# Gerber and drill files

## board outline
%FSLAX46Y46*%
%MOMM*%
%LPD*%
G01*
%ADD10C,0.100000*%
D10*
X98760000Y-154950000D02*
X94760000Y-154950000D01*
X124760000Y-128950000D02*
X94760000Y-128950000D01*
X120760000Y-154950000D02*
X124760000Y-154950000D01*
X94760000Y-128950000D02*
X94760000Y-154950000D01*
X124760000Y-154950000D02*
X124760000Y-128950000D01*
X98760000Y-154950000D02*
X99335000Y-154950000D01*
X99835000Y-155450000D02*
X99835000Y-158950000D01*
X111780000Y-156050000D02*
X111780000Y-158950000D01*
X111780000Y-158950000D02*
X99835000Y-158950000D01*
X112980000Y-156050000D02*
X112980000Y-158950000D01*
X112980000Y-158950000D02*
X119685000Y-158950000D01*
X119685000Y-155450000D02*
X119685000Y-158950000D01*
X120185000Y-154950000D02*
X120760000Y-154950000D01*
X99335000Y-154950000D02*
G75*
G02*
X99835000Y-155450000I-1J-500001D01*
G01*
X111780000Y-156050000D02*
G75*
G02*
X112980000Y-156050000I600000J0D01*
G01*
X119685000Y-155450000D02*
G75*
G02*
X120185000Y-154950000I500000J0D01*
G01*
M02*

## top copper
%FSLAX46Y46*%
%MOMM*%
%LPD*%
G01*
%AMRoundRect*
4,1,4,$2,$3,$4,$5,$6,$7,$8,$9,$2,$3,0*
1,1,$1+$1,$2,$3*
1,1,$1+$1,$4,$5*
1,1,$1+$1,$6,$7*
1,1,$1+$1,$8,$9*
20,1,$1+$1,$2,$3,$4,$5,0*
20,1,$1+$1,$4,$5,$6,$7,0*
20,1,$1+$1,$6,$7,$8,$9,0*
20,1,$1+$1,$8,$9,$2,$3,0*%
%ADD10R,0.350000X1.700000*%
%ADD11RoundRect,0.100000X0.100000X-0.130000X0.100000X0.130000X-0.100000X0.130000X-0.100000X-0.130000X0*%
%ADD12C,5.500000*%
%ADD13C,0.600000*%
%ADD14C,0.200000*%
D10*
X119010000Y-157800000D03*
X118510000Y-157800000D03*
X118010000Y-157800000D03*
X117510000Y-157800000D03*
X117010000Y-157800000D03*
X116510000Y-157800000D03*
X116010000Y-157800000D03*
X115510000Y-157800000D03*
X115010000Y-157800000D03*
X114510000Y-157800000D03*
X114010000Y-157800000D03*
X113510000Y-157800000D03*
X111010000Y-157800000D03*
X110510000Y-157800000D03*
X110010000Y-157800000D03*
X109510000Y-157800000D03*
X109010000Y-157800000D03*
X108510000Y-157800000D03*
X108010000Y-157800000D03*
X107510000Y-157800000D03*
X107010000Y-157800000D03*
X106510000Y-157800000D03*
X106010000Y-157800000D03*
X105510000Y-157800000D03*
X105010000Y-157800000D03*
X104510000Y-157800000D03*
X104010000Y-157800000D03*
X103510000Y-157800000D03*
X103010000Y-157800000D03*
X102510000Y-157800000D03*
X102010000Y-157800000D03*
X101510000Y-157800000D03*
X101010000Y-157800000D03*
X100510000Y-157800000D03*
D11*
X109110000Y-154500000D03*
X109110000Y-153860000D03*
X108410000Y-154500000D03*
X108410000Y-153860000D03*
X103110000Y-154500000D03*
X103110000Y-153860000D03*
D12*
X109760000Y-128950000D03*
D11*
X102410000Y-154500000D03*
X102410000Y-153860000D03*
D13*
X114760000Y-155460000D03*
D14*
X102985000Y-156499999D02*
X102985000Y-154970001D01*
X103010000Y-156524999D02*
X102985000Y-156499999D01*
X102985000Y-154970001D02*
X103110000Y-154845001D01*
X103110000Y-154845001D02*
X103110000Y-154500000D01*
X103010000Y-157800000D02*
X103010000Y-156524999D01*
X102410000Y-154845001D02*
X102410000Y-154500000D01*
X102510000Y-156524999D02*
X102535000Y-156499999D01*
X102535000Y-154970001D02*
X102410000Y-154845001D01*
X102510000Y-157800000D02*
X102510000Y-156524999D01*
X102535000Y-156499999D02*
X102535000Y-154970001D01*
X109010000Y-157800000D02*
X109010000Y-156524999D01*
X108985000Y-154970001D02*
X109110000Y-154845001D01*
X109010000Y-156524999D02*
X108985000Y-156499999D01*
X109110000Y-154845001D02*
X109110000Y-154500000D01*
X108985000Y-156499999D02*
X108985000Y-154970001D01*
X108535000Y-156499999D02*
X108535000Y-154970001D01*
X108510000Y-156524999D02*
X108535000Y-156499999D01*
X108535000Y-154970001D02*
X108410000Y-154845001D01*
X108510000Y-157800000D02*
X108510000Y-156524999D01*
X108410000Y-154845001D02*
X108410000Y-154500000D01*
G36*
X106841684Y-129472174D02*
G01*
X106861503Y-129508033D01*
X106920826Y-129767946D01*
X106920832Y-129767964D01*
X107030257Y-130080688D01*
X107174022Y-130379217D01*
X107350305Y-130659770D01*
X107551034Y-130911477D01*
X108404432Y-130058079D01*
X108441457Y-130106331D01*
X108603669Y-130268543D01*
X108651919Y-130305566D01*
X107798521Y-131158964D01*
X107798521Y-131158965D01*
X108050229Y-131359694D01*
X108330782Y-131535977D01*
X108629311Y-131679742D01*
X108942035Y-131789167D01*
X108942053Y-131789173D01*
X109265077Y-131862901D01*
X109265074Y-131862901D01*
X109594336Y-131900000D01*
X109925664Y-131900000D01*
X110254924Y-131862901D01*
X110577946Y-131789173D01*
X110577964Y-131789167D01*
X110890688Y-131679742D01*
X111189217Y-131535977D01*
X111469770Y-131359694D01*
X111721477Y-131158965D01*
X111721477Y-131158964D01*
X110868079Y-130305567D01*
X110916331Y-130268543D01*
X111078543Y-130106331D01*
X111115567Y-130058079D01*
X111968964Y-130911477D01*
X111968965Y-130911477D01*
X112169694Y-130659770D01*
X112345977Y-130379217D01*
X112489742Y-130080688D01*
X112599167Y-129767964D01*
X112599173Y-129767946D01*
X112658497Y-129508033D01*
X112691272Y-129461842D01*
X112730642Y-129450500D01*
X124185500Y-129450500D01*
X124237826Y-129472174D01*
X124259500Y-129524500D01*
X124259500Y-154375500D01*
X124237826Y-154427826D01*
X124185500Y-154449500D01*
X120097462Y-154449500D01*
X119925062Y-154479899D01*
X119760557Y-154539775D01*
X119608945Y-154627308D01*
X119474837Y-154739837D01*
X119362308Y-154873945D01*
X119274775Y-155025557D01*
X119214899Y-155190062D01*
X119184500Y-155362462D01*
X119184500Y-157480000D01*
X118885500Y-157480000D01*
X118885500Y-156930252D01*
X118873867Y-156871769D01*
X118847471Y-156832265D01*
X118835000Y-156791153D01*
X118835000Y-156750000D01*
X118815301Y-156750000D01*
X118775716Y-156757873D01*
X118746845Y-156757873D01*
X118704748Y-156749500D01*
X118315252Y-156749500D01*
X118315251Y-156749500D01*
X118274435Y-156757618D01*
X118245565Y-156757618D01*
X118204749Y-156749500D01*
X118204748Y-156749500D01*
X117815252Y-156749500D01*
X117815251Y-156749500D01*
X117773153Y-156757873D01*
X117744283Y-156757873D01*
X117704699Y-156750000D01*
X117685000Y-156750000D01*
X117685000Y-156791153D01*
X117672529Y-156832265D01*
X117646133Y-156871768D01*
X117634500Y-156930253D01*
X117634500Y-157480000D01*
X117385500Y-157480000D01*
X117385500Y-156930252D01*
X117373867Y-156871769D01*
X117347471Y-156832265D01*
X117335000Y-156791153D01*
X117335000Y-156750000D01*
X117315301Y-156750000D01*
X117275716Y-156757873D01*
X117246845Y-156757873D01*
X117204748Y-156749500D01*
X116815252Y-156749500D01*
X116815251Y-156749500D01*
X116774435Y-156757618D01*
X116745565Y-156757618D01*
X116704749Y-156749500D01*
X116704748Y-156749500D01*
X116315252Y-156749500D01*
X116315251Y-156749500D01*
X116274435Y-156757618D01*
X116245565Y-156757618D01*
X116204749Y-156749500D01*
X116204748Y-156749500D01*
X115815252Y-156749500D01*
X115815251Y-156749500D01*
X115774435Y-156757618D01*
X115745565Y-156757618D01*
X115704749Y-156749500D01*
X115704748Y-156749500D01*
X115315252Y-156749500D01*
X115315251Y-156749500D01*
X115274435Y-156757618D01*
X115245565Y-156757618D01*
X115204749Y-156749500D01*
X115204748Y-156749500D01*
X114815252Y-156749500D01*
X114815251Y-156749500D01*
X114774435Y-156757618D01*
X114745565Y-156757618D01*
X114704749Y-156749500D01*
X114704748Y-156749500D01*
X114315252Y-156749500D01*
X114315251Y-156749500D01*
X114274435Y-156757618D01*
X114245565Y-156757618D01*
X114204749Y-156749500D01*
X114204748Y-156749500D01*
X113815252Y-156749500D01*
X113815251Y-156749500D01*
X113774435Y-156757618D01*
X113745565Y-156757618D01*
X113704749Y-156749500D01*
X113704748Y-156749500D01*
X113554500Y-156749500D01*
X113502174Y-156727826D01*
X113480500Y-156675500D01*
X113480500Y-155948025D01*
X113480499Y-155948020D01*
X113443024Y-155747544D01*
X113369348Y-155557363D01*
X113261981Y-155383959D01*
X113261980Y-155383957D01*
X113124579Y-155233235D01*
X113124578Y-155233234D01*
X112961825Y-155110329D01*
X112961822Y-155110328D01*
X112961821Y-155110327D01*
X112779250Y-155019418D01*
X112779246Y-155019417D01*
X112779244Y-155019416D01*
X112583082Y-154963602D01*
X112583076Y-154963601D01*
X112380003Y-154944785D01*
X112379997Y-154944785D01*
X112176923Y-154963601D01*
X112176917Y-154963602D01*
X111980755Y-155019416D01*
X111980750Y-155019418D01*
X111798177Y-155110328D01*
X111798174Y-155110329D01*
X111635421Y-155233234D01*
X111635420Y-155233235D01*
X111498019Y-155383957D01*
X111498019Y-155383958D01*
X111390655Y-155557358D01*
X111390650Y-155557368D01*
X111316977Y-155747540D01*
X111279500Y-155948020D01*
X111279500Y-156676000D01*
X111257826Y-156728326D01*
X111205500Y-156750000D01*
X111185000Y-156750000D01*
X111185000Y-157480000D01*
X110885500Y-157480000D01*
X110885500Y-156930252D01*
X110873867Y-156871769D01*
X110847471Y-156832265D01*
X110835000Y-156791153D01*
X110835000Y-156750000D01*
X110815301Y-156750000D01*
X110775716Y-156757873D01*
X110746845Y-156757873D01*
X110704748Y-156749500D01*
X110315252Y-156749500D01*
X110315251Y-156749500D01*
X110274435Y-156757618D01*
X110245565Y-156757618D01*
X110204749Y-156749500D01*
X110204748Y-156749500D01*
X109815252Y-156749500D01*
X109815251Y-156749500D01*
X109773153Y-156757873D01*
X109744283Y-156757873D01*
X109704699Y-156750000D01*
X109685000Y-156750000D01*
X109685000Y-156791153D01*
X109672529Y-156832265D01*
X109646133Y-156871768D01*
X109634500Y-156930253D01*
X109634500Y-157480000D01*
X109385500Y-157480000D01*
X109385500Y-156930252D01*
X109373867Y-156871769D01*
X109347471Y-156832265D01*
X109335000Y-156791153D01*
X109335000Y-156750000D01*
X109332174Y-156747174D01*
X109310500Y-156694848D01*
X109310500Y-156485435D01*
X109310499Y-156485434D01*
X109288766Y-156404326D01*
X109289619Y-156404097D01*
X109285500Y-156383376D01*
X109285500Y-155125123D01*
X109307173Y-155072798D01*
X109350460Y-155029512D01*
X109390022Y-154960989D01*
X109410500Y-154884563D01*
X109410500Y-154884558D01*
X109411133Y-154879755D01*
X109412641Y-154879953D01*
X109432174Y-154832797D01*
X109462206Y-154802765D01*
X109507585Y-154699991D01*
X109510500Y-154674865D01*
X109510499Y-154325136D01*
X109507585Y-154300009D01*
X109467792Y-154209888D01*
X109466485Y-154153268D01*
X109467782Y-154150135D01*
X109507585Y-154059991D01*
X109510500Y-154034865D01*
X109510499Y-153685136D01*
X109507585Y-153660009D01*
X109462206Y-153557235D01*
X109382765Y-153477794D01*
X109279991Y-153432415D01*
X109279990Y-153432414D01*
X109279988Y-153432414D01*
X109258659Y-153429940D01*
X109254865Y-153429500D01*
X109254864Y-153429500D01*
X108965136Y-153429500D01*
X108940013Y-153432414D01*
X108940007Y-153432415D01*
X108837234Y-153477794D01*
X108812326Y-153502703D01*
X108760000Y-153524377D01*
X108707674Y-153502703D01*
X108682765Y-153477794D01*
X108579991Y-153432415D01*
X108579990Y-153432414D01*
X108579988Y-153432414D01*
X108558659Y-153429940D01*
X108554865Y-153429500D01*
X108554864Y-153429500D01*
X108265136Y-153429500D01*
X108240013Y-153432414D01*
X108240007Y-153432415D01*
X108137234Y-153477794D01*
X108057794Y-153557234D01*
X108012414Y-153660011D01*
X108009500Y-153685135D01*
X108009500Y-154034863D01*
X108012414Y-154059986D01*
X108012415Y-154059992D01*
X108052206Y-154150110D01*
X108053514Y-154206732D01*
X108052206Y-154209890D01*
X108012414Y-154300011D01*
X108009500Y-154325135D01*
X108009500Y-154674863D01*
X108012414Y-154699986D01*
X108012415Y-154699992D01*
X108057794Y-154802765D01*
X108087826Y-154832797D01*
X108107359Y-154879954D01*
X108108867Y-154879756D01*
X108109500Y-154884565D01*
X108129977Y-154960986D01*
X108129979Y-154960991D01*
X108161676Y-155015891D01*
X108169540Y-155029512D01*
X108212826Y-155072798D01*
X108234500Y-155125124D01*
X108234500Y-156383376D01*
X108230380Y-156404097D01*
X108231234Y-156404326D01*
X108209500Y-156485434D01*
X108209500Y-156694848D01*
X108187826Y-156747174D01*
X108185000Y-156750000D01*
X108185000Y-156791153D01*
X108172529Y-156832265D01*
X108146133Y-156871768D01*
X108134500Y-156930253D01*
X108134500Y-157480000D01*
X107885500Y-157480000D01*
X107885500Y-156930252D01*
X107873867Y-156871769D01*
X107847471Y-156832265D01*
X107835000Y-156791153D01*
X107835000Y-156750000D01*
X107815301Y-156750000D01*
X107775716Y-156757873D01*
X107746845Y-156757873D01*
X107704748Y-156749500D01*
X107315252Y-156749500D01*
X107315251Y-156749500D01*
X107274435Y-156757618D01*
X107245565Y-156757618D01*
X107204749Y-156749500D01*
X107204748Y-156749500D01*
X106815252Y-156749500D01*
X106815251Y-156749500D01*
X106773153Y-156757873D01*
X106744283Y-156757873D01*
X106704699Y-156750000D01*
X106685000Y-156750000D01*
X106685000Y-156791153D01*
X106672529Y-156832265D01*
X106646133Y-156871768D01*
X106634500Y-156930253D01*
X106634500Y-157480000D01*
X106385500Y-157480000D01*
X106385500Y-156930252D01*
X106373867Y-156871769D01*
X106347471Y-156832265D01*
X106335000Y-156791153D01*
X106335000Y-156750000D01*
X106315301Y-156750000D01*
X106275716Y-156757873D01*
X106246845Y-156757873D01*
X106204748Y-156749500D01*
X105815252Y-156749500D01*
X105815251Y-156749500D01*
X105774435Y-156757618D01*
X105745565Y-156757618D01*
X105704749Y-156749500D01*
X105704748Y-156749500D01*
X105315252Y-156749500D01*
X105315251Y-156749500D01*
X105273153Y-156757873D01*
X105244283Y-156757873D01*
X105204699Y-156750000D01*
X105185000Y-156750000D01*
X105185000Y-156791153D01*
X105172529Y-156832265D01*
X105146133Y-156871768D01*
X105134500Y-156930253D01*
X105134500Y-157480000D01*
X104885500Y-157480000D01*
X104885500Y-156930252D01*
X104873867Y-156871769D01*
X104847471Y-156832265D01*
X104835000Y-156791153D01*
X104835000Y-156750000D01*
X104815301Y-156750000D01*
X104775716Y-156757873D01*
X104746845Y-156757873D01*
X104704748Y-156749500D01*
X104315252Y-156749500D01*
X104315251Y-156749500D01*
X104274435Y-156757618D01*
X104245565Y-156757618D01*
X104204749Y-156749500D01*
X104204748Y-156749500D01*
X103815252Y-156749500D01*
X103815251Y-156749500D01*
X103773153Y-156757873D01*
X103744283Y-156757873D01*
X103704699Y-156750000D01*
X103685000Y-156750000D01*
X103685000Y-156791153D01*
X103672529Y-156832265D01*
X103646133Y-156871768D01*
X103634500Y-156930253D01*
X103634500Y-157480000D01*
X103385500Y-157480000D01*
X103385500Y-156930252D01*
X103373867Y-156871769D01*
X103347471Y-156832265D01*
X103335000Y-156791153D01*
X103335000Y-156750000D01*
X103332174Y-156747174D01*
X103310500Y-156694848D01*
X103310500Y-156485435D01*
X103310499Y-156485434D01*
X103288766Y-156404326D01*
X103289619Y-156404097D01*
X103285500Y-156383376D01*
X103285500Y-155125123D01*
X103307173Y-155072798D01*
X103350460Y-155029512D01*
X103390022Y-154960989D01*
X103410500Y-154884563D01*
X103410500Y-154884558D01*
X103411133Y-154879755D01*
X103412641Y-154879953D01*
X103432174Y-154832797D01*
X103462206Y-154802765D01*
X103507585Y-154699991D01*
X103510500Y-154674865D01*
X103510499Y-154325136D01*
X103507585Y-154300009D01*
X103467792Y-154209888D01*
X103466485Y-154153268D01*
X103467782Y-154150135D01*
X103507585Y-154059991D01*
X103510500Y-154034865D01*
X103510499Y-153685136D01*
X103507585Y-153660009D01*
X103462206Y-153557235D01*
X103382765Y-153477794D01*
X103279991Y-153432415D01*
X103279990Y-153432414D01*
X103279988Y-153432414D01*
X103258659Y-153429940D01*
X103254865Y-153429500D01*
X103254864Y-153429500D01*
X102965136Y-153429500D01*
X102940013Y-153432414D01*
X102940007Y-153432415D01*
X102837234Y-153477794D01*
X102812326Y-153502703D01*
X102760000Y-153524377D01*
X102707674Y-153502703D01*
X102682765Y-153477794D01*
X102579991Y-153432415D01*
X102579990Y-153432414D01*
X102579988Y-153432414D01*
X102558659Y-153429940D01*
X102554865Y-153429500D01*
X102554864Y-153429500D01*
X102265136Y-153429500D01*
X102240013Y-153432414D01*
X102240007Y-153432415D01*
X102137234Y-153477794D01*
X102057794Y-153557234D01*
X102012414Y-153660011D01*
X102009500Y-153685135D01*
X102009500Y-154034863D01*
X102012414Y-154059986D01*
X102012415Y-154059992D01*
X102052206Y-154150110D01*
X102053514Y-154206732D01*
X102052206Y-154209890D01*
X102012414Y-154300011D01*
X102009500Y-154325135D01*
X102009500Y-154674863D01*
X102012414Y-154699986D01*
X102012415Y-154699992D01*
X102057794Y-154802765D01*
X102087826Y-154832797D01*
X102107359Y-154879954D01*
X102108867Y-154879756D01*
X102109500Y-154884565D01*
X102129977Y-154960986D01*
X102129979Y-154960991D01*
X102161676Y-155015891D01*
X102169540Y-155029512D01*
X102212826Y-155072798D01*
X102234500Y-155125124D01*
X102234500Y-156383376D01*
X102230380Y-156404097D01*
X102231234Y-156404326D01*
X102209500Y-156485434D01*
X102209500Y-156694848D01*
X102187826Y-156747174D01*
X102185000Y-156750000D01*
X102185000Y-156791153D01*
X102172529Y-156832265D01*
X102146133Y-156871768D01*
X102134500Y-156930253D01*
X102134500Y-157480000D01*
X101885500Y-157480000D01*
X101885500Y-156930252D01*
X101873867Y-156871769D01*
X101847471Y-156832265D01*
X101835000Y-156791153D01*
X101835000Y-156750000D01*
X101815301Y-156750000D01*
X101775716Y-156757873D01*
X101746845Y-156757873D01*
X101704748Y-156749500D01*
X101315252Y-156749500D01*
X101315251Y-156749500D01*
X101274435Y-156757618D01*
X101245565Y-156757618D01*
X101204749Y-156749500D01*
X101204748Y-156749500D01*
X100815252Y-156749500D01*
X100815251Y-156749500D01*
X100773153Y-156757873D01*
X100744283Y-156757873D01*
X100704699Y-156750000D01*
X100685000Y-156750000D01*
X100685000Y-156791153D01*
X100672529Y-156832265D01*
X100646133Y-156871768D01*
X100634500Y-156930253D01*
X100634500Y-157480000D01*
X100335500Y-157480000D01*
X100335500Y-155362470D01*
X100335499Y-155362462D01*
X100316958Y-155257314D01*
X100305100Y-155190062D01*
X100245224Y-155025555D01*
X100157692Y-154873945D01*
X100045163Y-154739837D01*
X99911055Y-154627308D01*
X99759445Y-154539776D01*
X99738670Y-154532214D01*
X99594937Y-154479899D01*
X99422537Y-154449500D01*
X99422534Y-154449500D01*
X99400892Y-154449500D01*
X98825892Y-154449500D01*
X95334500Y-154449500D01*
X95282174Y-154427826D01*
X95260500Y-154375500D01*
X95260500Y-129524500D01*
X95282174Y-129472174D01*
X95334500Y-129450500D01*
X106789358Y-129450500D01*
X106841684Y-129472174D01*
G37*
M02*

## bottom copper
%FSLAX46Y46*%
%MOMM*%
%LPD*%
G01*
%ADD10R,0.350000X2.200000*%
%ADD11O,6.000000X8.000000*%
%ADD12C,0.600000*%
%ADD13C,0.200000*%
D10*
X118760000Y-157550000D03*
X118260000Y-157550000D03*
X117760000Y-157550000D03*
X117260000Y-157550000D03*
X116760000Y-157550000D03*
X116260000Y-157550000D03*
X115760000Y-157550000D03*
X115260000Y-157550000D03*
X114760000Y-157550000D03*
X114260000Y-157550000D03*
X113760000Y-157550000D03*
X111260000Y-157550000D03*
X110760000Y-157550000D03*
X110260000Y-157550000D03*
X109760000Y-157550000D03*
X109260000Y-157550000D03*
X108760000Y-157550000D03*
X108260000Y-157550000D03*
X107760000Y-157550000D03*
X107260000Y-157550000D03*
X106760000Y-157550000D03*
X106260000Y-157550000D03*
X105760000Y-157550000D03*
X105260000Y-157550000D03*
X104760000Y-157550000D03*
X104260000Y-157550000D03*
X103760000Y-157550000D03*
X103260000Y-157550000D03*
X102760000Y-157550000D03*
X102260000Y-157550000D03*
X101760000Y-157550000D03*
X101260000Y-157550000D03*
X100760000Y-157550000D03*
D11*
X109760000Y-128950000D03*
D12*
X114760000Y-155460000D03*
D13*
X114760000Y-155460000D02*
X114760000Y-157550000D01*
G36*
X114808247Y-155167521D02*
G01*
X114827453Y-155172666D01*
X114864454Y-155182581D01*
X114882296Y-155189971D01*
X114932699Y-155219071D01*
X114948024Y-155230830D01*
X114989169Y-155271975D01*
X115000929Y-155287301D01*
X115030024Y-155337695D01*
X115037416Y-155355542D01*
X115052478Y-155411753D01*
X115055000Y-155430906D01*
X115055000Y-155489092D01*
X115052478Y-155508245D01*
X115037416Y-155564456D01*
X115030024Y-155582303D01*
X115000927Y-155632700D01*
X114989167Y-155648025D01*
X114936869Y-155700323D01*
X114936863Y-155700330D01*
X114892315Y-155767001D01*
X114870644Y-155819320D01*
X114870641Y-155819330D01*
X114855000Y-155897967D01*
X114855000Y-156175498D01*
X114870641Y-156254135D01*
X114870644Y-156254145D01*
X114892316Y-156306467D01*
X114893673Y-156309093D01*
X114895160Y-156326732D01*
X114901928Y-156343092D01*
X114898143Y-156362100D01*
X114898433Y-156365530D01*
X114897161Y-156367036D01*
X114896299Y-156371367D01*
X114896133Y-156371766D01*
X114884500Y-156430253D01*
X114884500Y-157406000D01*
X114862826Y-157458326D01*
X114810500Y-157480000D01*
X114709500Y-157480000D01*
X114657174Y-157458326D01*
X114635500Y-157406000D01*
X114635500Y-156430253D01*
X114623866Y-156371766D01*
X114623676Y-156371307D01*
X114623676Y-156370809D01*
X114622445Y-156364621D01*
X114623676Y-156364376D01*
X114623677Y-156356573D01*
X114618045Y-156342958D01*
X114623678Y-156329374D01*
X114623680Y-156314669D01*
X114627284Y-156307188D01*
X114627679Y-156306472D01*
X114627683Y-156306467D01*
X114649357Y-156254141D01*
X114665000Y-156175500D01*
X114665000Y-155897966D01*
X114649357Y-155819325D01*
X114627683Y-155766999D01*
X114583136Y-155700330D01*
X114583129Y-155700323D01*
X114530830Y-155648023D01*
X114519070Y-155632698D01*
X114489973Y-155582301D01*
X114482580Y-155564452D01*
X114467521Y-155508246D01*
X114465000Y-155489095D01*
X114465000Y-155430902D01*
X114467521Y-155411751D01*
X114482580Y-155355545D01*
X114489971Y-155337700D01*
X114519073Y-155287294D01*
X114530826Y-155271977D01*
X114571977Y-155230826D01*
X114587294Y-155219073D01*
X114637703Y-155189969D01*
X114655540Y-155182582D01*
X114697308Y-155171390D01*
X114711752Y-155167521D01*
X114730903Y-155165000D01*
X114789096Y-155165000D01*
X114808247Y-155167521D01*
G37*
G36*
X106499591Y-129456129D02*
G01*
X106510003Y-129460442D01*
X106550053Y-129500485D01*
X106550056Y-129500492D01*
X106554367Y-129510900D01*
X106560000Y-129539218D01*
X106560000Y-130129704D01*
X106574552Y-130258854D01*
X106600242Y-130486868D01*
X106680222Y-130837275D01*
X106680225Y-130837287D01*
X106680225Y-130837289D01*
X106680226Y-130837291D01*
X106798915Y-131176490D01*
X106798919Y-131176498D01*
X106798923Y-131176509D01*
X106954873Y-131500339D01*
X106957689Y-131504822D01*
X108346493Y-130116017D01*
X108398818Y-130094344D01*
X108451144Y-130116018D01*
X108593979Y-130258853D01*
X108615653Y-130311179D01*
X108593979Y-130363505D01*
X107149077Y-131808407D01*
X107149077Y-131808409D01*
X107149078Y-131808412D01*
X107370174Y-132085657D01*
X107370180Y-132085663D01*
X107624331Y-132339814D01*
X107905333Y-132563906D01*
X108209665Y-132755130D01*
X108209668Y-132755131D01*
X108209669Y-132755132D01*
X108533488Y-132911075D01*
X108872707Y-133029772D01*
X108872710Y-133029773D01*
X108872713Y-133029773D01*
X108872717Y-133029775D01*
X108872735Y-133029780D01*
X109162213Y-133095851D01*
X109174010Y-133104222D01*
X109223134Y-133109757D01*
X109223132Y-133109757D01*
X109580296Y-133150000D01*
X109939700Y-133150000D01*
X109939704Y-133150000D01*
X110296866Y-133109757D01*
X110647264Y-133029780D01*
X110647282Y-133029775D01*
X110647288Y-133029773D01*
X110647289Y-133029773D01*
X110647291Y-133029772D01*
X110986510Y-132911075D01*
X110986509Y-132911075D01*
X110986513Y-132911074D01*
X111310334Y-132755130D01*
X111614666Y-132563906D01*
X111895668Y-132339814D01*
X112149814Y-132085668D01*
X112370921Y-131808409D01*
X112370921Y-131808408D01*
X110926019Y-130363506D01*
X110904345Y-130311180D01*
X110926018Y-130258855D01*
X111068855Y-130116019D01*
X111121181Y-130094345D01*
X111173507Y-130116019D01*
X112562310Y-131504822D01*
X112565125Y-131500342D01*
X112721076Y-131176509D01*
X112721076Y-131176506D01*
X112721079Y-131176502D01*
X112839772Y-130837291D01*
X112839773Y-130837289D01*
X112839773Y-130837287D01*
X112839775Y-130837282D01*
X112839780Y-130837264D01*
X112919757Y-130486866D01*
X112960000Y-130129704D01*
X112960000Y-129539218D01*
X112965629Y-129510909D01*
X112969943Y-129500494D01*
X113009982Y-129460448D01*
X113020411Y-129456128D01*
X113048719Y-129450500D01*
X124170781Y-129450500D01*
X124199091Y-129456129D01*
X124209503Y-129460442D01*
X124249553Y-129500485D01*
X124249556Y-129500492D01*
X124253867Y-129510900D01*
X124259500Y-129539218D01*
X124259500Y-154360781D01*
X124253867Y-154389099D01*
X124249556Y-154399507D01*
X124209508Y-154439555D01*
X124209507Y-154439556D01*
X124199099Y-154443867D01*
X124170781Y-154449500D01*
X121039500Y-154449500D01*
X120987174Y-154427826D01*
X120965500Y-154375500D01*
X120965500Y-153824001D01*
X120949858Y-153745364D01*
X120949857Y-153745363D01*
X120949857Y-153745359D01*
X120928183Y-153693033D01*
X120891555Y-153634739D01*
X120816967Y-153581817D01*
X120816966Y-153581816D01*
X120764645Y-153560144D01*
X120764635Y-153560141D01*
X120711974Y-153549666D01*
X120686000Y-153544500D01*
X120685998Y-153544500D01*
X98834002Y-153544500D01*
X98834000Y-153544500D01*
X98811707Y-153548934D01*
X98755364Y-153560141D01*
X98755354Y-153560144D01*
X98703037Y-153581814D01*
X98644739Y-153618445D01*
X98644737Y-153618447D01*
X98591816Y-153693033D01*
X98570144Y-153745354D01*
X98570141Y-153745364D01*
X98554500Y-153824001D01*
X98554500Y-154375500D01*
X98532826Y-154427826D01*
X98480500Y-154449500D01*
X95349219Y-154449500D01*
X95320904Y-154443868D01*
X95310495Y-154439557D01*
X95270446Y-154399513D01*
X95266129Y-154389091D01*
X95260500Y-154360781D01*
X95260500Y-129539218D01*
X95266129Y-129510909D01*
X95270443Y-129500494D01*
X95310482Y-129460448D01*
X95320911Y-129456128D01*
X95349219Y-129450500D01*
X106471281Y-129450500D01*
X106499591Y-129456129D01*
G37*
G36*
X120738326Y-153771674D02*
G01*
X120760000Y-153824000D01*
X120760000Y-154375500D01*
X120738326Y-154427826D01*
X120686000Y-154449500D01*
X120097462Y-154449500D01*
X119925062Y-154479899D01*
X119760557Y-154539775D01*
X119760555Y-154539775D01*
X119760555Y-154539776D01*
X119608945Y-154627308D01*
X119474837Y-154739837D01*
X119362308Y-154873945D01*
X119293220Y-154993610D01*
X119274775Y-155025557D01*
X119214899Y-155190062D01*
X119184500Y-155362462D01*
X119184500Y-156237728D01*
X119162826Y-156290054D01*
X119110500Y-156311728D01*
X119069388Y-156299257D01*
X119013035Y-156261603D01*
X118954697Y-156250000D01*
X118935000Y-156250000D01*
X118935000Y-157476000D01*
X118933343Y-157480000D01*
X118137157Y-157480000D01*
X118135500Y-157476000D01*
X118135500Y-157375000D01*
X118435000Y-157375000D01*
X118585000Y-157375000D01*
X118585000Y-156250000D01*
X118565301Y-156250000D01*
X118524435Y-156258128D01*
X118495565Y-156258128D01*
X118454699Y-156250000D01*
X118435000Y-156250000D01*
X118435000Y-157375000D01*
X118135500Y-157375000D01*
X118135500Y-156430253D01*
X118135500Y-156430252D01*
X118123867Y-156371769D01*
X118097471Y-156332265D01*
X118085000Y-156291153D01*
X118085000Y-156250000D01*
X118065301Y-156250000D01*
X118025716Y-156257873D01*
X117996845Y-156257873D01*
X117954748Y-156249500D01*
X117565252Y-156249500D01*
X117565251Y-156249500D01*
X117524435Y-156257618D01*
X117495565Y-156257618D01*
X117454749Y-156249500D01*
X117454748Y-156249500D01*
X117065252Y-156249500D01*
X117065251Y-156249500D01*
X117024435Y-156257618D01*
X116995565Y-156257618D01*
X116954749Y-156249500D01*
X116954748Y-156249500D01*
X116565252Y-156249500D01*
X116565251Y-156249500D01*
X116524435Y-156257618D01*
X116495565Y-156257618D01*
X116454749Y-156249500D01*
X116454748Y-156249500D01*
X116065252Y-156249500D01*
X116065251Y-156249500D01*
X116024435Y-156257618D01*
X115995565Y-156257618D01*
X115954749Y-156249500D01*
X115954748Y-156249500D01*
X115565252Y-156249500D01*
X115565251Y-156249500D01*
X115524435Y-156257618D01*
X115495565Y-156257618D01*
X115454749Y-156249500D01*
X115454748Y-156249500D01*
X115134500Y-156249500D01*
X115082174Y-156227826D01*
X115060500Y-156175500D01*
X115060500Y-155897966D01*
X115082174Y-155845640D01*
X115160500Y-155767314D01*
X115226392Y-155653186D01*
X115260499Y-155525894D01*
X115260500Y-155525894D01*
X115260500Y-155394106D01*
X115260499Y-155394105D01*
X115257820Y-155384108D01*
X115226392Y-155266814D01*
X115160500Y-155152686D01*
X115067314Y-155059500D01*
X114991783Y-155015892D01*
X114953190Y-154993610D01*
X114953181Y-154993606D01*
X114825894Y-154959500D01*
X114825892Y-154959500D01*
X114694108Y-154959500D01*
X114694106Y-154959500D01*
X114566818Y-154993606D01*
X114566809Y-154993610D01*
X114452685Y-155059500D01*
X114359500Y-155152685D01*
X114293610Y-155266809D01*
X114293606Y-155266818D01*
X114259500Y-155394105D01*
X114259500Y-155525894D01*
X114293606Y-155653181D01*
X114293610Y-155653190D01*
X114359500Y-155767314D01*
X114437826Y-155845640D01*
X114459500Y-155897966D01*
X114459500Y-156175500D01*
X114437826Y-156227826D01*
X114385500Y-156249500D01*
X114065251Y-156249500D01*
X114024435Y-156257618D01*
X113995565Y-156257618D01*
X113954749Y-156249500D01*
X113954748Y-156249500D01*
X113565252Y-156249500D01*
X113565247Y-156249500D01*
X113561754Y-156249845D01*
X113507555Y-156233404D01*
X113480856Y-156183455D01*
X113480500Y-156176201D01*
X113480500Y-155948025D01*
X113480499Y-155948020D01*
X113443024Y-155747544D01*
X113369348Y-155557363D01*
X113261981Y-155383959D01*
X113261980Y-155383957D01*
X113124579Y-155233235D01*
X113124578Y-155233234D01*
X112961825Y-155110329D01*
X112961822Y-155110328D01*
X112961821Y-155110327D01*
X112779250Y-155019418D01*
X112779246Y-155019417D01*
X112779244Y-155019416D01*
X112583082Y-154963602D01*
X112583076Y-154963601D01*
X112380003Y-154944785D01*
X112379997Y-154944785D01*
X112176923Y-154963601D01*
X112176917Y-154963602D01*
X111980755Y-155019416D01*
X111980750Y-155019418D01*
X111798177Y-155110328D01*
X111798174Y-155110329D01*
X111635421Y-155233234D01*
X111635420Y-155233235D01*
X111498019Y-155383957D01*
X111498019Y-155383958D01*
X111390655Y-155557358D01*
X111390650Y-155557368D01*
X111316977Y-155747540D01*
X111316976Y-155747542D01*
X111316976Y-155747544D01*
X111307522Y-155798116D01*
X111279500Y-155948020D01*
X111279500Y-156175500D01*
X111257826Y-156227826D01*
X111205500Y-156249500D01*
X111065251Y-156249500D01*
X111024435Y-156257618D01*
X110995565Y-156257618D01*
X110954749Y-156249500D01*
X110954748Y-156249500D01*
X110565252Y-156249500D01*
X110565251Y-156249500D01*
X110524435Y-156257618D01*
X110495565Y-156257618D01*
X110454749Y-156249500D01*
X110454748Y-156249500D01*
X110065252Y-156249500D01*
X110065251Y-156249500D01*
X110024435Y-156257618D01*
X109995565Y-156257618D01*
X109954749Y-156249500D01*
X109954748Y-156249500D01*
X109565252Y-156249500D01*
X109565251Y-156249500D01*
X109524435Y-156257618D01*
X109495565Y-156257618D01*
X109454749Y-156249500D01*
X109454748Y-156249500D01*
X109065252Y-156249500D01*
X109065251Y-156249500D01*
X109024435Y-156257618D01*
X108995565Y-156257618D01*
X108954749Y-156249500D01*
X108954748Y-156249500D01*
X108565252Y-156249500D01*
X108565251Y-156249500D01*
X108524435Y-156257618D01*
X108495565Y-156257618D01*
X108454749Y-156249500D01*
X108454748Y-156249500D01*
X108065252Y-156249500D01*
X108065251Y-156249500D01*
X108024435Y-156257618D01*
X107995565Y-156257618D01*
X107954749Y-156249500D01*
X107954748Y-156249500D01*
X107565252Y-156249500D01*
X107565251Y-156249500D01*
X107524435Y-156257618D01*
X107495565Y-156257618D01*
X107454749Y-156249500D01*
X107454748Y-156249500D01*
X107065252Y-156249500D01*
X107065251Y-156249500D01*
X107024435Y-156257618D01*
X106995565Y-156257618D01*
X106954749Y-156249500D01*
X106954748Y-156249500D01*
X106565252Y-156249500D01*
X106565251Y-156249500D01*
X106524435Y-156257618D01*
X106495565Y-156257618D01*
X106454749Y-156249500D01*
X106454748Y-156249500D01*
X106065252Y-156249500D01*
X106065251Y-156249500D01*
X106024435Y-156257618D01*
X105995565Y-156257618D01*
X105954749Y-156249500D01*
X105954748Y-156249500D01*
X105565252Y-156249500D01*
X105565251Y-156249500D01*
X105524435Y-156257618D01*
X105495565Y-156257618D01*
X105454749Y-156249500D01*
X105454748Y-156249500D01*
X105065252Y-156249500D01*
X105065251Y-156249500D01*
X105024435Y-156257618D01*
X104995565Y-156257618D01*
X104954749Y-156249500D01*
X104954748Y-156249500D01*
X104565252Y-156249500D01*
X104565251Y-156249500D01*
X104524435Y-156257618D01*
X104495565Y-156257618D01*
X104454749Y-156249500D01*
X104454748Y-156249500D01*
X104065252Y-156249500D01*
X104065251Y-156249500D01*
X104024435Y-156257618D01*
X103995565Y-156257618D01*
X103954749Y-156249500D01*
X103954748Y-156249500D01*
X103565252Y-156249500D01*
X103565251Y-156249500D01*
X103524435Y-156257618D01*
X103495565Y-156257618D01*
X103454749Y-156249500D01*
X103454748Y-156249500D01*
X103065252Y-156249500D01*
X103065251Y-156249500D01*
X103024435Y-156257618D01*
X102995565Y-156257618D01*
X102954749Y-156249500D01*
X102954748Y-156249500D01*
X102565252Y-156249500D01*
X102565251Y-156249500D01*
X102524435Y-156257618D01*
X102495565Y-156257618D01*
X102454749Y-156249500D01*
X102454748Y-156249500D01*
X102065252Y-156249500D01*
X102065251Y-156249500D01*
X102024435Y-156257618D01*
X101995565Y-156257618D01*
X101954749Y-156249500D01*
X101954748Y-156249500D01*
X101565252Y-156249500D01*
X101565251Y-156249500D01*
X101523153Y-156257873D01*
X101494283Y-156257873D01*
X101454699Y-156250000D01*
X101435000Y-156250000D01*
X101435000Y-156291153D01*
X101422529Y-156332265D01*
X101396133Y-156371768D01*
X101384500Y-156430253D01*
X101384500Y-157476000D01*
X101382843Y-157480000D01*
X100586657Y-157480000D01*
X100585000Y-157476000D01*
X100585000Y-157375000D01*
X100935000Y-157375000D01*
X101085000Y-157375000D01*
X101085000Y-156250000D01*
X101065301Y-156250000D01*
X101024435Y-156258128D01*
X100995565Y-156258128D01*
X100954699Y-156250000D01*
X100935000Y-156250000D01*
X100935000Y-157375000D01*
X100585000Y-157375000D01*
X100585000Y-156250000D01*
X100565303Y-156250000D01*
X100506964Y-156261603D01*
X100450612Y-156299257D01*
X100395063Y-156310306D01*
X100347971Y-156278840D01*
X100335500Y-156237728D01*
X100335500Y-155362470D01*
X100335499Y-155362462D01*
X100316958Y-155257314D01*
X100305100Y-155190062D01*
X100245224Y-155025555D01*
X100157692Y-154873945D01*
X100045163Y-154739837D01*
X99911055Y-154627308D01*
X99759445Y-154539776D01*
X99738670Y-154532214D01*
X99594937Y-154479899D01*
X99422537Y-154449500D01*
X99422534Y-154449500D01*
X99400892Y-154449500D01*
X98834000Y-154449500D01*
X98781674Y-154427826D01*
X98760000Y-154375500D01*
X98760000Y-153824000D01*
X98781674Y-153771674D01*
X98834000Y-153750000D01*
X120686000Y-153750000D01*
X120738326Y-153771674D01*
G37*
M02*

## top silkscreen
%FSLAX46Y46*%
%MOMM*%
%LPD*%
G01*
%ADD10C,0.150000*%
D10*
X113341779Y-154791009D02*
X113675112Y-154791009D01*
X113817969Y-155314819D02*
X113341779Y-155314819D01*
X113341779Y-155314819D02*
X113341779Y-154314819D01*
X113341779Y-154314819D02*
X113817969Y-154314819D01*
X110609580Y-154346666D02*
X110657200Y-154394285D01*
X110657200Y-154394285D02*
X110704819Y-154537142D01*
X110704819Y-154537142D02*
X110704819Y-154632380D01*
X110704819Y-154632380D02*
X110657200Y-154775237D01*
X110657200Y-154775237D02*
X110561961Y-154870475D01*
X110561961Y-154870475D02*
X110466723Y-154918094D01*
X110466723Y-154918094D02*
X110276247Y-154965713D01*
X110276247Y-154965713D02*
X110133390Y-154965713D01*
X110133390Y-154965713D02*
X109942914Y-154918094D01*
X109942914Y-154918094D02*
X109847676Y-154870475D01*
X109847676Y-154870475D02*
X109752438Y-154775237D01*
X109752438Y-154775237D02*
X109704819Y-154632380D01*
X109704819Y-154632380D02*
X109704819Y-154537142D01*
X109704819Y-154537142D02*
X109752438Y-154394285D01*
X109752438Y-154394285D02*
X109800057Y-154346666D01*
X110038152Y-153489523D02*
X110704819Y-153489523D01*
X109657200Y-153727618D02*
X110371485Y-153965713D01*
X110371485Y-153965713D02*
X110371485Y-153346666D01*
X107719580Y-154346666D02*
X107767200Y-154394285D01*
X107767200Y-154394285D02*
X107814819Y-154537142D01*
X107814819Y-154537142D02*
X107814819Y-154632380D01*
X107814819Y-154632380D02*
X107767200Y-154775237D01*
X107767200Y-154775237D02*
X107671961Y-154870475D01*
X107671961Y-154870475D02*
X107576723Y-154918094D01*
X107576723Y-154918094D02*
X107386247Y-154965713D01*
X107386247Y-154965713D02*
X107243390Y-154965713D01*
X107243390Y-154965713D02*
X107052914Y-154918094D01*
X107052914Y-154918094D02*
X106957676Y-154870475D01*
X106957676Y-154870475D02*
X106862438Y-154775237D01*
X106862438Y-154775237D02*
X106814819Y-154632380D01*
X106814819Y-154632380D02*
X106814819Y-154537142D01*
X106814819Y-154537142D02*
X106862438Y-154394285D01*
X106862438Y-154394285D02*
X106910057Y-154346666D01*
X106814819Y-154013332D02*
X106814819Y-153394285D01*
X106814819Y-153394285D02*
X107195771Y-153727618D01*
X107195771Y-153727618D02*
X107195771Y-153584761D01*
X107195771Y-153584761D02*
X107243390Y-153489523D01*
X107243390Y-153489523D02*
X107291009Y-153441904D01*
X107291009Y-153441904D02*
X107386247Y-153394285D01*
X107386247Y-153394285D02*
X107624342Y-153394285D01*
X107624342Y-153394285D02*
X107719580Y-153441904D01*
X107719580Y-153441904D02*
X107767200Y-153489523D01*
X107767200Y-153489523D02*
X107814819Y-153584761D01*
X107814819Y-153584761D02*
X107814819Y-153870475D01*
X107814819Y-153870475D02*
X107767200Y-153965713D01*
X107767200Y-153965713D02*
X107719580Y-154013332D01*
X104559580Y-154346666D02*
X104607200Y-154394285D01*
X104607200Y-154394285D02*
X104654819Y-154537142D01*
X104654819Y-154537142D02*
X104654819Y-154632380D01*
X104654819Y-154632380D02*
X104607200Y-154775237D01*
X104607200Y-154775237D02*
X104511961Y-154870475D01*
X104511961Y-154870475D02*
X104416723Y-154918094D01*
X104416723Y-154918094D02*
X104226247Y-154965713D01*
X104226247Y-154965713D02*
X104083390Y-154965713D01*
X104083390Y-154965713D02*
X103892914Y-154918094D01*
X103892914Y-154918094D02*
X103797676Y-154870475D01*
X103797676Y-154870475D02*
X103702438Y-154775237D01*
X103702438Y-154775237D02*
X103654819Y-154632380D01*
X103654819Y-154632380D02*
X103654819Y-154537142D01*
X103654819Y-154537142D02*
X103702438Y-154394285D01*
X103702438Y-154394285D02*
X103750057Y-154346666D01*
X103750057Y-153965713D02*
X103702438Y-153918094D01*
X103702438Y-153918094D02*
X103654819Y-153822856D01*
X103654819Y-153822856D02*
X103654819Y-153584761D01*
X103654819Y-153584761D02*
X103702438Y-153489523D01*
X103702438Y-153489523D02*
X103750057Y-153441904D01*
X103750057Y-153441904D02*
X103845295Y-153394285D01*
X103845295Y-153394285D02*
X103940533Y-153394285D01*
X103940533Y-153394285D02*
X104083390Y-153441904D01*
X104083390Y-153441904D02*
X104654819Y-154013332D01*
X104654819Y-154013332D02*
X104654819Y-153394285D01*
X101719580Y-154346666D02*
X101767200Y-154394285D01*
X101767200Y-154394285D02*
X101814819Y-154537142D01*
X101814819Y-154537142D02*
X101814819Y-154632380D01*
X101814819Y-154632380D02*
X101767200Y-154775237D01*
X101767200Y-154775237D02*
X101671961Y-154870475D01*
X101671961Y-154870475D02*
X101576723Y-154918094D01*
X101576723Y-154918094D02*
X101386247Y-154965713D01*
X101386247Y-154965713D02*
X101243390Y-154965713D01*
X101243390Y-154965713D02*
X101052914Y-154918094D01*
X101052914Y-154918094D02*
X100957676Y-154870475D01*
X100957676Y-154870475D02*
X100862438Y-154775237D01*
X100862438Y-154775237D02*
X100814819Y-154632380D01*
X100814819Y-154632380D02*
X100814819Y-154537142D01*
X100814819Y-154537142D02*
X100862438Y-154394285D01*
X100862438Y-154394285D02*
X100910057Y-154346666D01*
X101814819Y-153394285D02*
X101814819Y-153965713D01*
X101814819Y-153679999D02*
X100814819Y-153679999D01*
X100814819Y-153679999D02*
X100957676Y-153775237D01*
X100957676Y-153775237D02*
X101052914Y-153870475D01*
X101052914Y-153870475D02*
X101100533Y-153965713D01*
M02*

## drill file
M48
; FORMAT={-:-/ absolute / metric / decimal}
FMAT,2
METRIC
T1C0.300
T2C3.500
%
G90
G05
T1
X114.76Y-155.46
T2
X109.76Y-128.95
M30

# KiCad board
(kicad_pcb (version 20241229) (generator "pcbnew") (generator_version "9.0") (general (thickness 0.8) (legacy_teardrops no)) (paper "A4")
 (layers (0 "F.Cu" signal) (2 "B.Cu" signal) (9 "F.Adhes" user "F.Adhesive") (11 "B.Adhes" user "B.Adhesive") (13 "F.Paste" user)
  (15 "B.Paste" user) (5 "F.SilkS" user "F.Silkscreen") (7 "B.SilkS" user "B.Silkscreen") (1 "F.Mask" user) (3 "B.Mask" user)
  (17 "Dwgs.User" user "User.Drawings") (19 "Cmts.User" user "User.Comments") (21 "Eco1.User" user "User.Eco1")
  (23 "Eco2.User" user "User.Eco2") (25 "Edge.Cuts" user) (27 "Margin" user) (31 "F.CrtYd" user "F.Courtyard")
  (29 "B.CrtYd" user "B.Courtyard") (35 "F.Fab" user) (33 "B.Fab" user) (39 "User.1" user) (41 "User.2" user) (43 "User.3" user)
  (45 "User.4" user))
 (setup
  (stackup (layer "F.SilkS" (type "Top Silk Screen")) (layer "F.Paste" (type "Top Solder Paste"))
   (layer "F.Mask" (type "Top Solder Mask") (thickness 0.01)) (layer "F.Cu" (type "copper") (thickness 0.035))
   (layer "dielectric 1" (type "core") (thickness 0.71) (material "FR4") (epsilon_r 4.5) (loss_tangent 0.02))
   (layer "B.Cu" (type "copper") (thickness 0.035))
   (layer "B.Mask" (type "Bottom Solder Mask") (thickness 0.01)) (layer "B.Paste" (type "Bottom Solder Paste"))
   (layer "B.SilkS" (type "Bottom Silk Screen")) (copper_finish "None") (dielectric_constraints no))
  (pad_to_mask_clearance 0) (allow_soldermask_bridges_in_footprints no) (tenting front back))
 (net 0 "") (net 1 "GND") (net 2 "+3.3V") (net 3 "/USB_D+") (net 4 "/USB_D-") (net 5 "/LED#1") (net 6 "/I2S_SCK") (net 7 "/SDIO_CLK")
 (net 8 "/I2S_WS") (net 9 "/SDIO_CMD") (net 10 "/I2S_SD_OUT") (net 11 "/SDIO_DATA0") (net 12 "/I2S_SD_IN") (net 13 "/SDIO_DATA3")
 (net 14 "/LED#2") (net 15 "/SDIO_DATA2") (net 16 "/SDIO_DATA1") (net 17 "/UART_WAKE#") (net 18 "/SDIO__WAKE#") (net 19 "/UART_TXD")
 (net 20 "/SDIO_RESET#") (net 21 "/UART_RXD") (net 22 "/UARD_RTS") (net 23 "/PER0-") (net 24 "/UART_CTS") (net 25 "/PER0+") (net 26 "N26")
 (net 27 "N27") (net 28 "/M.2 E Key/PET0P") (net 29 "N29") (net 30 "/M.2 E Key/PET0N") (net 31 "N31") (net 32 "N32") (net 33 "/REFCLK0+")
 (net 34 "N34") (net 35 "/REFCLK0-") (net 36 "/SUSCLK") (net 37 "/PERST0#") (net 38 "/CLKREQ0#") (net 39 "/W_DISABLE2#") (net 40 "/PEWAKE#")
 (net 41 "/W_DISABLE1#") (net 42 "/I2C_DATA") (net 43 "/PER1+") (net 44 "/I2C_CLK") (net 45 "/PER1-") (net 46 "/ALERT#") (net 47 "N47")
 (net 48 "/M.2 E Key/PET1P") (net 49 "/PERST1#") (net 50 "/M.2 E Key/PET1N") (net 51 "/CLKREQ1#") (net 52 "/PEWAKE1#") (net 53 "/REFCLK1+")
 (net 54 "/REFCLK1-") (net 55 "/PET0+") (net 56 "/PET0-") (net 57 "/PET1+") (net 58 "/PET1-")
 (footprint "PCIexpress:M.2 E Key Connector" (layer "F.Cu") (at 109.76 157.84)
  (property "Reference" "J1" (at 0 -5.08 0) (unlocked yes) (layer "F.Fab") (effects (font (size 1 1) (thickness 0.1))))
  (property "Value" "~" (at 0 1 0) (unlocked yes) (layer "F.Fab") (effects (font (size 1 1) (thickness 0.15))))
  (fp_line (start -11 -2.89) (end -10.425 -2.89) (stroke (width 0.1) (type default)) (layer "Edge.Cuts"))
  (fp_line (start -9.925 -2.39) (end -9.925 1.11) (stroke (width 0.1) (type default)) (layer "Edge.Cuts"))
  (fp_line (start 2.02 -1.79) (end 2.02 1.11) (stroke (width 0.1) (type default)) (layer "Edge.Cuts"))
  (fp_line (start 2.02 1.11) (end -9.925 1.11) (stroke (width 0.1) (type default)) (layer "Edge.Cuts"))
  (fp_line (start 3.22 -1.79) (end 3.22 1.11) (stroke (width 0.1) (type default)) (layer "Edge.Cuts"))
  (fp_line (start 3.22 1.11) (end 9.925 1.11) (stroke (width 0.1) (type default)) (layer "Edge.Cuts"))
  (fp_line (start 9.925 -2.39) (end 9.925 1.11) (stroke (width 0.1) (type default)) (layer "Edge.Cuts"))
  (fp_line (start 10.425 -2.89) (end 11 -2.89) (stroke (width 0.1) (type default)) (layer "Edge.Cuts"))
  (fp_arc (start -10.425 -2.89) (mid -10.071447 -2.743553) (end -9.925 -2.39) (stroke (width 0.1) (type default)) (layer "Edge.Cuts"))
  (fp_arc (start 2.02 -1.79) (mid 2.62 -2.39) (end 3.22 -1.79) (stroke (width 0.1) (type default)) (layer "Edge.Cuts"))
  (fp_arc (start 9.925 -2.39) (mid 10.071447 -2.743553) (end 10.425 -2.89) (stroke (width 0.1) (type default)) (layer "Edge.Cuts"))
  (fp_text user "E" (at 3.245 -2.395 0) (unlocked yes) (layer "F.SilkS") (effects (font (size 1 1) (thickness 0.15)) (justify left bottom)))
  (pad "1" smd rect (at 9.25 -0.04 180) (size 0.35 1.7) (layers "F.Cu") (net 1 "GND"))
  (pad "2" smd rect (at 9 -0.29 180) (size 0.35 2.2) (layers "B.Cu") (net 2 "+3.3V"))
  (pad "3" smd rect (at 8.75 -0.04 180) (size 0.35 1.7) (layers "F.Cu") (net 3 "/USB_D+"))
  (pad "4" smd rect (at 8.5 -0.29 180) (size 0.35 2.2) (layers "B.Cu") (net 2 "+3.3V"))
  (pad "5" smd rect (at 8.25 -0.04 180) (size 0.35 1.7) (layers "F.Cu") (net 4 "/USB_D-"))
  (pad "6" smd rect (at 8 -0.29 180) (size 0.35 2.2) (layers "B.Cu") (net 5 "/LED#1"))
  (pad "7" smd rect (at 7.75 -0.04 180) (size 0.35 1.7) (layers "F.Cu") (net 1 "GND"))
  (pad "8" smd rect (at 7.5 -0.29 180) (size 0.35 2.2) (layers "B.Cu") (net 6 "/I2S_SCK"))
  (pad "9" smd rect (at 7.25 -0.04 180) (size 0.35 1.7) (layers "F.Cu") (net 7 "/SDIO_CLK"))
  (pad "10" smd rect (at 7 -0.29 180) (size 0.35 2.2) (layers "B.Cu") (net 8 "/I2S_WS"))
  (pad "11" smd rect (at 6.75 -0.04 180) (size 0.35 1.7) (layers "F.Cu") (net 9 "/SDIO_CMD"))
  (pad "12" smd rect (at 6.5 -0.29 180) (size 0.35 2.2) (layers "B.Cu") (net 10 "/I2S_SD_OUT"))
  (pad "13" smd rect (at 6.25 -0.04 180) (size 0.35 1.7) (layers "F.Cu") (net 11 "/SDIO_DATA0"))
  (pad "14" smd rect (at 6 -0.29 180) (size 0.35 2.2) (layers "B.Cu") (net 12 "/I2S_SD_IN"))
  (pad "15" smd rect (at 5.75 -0.04 180) (size 0.35 1.7) (layers "F.Cu") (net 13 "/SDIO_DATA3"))
  (pad "16" smd rect (at 5.5 -0.29 180) (size 0.35 2.2) (layers "B.Cu") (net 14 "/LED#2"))
  (pad "17" smd rect (at 5.25 -0.04 180) (size 0.35 1.7) (layers "F.Cu") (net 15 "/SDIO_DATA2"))
  (pad "18" smd rect (at 5 -0.29 180) (size 0.35 2.2) (layers "B.Cu") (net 1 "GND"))
  (pad "19" smd rect (at 4.75 -0.04 180) (size 0.35 1.7) (layers "F.Cu") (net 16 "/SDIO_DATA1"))
  (pad "20" smd rect (at 4.5 -0.29 180) (size 0.35 2.2) (layers "B.Cu") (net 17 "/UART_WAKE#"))
  (pad "21" smd rect (at 4.25 -0.04 180) (size 0.35 1.7) (layers "F.Cu") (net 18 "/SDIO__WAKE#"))
  (pad "22" smd rect (at 4 -0.29 180) (size 0.35 2.2) (layers "B.Cu") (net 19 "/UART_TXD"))
  (pad "23" smd rect (at 3.75 -0.04 180) (size 0.35 1.7) (layers "F.Cu") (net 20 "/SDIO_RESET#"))
  (pad "32" smd rect (at 1.5 -0.29 180) (size 0.35 2.2) (layers "B.Cu") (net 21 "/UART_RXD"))
  (pad "33" smd rect (at 1.25 -0.04 180) (size 0.35 1.7) (layers "F.Cu") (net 1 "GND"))
  (pad "34" smd rect (at 1 -0.29 180) (size 0.35 2.2) (layers "B.Cu") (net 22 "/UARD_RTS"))
  (pad "35" smd rect (at 0.75 -0.04 180) (size 0.35 1.7) (layers "F.Cu") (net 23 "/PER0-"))
  (pad "36" smd rect (at 0.5 -0.29 180) (size 0.35 2.2) (layers "B.Cu") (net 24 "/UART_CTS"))
  (pad "37" smd rect (at 0.25 -0.04 180) (size 0.35 1.7) (layers "F.Cu") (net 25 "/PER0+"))
  (pad "38" smd rect (at 0 -0.29 180) (size 0.35 2.2) (layers "B.Cu") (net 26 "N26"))
  (pad "39" smd rect (at -0.25 -0.04 180) (size 0.35 1.7) (layers "F.Cu") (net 1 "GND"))
  (pad "40" smd rect (at -0.5 -0.29 180) (size 0.35 2.2) (layers "B.Cu") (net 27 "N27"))
  (pad "41" smd rect (at -0.75 -0.04 180) (size 0.35 1.7) (layers "F.Cu") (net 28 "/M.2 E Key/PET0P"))
  (pad "42" smd rect (at -1 -0.29 180) (size 0.35 2.2) (layers "B.Cu") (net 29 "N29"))
  (pad "43" smd rect (at -1.25 -0.04 180) (size 0.35 1.7) (layers "F.Cu") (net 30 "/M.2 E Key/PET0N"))
  (pad "44" smd rect (at -1.5 -0.29 180) (size 0.35 2.2) (layers "B.Cu") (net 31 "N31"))
  (pad "45" smd rect (at -1.75 -0.04 180) (size 0.35 1.7) (layers "F.Cu") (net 1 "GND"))
  (pad "46" smd rect (at -2 -0.29 180) (size 0.35 2.2) (layers "B.Cu") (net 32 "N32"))
  (pad "47" smd rect (at -2.25 -0.04 180) (size 0.35 1.7) (layers "F.Cu") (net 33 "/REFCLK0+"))
  (pad "48" smd rect (at -2.5 -0.29 180) (size 0.35 2.2) (layers "B.Cu") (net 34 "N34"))
  (pad "49" smd rect (at -2.75 -0.04 180) (size 0.35 1.7) (layers "F.Cu") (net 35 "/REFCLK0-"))
  (pad "50" smd rect (at -3 -0.29 180) (size 0.35 2.2) (layers "B.Cu") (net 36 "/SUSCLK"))
  (pad "51" smd rect (at -3.25 -0.04 180) (size 0.35 1.7) (layers "F.Cu") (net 1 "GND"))
  (pad "52" smd rect (at -3.5 -0.29 180) (size 0.35 2.2) (layers "B.Cu") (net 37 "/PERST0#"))
  (pad "53" smd rect (at -3.75 -0.04 180) (size 0.35 1.7) (layers "F.Cu") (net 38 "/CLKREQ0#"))
  (pad "54" smd rect (at -4 -0.29 180) (size 0.35 2.2) (layers "B.Cu") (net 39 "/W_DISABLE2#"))
  (pad "55" smd rect (at -4.25 -0.04 180) (size 0.35 1.7) (layers "F.Cu") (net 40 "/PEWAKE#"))
  (pad "56" smd rect (at -4.5 -0.29 180) (size 0.35 2.2) (layers "B.Cu") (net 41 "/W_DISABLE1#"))
  (pad "57" smd rect (at -4.75 -0.04 180) (size 0.35 1.7) (layers "F.Cu") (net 1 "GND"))
  (pad "58" smd rect (at -5 -0.29 180) (size 0.35 2.2) (layers "B.Cu") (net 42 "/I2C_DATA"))
  (pad "59" smd rect (at -5.25 -0.04 180) (size 0.35 1.7) (layers "F.Cu") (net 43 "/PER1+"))
  (pad "60" smd rect (at -5.5 -0.29 180) (size 0.35 2.2) (layers "B.Cu") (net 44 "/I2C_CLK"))
  (pad "61" smd rect (at -5.75 -0.04 180) (size 0.35 1.7) (layers "F.Cu") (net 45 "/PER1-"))
  (pad "62" smd rect (at -6 -0.29 180) (size 0.35 2.2) (layers "B.Cu") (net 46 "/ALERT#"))
  (pad "63" smd rect (at -6.25 -0.04 180) (size 0.35 1.7) (layers "F.Cu") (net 1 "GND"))
  (pad "64" smd rect (at -6.5 -0.29 180) (size 0.35 2.2) (layers "B.Cu") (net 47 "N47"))
  (pad "65" smd rect (at -6.75 -0.04 180) (size 0.35 1.7) (layers "F.Cu") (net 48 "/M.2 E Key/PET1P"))
  (pad "66" smd rect (at -7 -0.29 180) (size 0.35 2.2) (layers "B.Cu") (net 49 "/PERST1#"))
  (pad "67" smd rect (at -7.25 -0.04 180) (size 0.35 1.7) (layers "F.Cu") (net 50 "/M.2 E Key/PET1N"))
  (pad "68" smd rect (at -7.5 -0.29 180) (size 0.35 2.2) (layers "B.Cu") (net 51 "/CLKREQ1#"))
  (pad "69" smd rect (at -7.75 -0.04 180) (size 0.35 1.7) (layers "F.Cu") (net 1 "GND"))
  (pad "70" smd rect (at -8 -0.29 180) (size 0.35 2.2) (layers "B.Cu") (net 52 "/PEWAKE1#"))
  (pad "71" smd rect (at -8.25 -0.04 180) (size 0.35 1.7) (layers "F.Cu") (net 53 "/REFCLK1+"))
  (pad "72" smd rect (at -8.5 -0.29 180) (size 0.35 2.2) (layers "B.Cu") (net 2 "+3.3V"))
  (pad "73" smd rect (at -8.75 -0.04 180) (size 0.35 1.7) (layers "F.Cu") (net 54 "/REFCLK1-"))
  (pad "74" smd rect (at -9 -0.29 180) (size 0.35 2.2) (layers "B.Cu") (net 2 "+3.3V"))
  (pad "75" smd rect (at -9.25 -0.04 180) (size 0.35 1.7) (layers "F.Cu") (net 1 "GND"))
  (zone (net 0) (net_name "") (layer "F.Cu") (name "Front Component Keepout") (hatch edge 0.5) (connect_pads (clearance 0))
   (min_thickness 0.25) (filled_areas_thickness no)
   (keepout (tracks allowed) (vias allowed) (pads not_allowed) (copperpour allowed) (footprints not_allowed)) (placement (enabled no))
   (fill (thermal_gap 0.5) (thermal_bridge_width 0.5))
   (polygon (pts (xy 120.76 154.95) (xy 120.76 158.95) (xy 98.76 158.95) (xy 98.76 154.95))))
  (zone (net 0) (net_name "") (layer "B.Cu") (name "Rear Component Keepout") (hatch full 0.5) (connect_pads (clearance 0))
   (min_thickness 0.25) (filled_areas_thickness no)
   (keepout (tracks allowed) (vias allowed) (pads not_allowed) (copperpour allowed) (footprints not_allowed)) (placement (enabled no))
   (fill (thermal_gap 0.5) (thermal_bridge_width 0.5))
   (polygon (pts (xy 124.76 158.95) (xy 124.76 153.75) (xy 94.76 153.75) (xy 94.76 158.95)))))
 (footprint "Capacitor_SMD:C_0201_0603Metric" (layer "F.Cu") (at 109.11 154.18 90)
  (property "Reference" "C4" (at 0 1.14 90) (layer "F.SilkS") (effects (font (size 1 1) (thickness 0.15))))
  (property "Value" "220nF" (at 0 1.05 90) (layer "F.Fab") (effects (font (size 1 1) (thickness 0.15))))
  (pad "" smd roundrect (at -0.345 0 90) (size 0.318 0.36) (layers "F.Paste") (roundrect_rratio 0.25))
  (pad "" smd roundrect (at 0.345 0 90) (size 0.318 0.36) (layers "F.Paste") (roundrect_rratio 0.25))
  (pad "1" smd roundrect (at -0.32 0 90) (size 0.46 0.4) (layers "F.Cu" "F.Mask") (roundrect_rratio 0.25) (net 28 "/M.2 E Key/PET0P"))
  (pad "2" smd roundrect (at 0.32 0 90) (size 0.46 0.4) (layers "F.Cu" "F.Mask") (roundrect_rratio 0.25) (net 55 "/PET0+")))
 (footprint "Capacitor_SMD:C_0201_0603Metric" (layer "F.Cu") (at 108.41 154.18 90)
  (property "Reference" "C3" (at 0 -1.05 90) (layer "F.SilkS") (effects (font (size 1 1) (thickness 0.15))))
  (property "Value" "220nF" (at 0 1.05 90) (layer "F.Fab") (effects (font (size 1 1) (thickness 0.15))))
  (pad "" smd roundrect (at -0.345 0 90) (size 0.318 0.36) (layers "F.Paste") (roundrect_rratio 0.25))
  (pad "" smd roundrect (at 0.345 0 90) (size 0.318 0.36) (layers "F.Paste") (roundrect_rratio 0.25))
  (pad "1" smd roundrect (at -0.32 0 90) (size 0.46 0.4) (layers "F.Cu" "F.Mask") (roundrect_rratio 0.25) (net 30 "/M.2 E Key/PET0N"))
  (pad "2" smd roundrect (at 0.32 0 90) (size 0.46 0.4) (layers "F.Cu" "F.Mask") (roundrect_rratio 0.25) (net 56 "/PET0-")))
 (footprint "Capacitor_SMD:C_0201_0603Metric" (layer "F.Cu") (at 103.11 154.18 90)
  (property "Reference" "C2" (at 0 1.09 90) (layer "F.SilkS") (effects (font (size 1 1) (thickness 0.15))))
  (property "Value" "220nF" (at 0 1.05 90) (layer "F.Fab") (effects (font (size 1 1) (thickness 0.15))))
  (pad "" smd roundrect (at -0.345 0 90) (size 0.318 0.36) (layers "F.Paste") (roundrect_rratio 0.25))
  (pad "" smd roundrect (at 0.345 0 90) (size 0.318 0.36) (layers "F.Paste") (roundrect_rratio 0.25))
  (pad "1" smd roundrect (at -0.32 0 90) (size 0.46 0.4) (layers "F.Cu" "F.Mask") (roundrect_rratio 0.25) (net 48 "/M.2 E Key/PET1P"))
  (pad "2" smd roundrect (at 0.32 0 90) (size 0.46 0.4) (layers "F.Cu" "F.Mask") (roundrect_rratio 0.25) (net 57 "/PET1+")))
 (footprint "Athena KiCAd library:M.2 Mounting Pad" (layer "F.Cu") (at 109.76 128.95)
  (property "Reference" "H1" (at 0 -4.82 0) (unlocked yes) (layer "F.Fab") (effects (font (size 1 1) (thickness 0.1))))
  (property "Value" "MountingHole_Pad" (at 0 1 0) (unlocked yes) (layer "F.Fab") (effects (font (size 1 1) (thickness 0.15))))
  (pad "1" thru_hole circle (at 0 0) (size 5.5 5.5) (drill 3.5) (layers "*.Cu" "*.Mask") (remove_unused_layers no) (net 1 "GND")
   (padstack (mode front_inner_back)
    (layer "Inner" (shape circle) (size 5.5 5.5) (zone_connect -1))
    (layer "B.Cu" (shape oval) (size 6 8) (thermal_bridge_angle 45) (zone_connect -1)))))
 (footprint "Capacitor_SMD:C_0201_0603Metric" (layer "F.Cu") (at 102.41 154.18 90)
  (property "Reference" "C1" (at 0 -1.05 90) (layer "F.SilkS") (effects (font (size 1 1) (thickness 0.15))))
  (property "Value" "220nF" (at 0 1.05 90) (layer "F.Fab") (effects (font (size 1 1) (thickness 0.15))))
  (pad "" smd roundrect (at -0.345 0 90) (size 0.318 0.36) (layers "F.Paste") (roundrect_rratio 0.25))
  (pad "" smd roundrect (at 0.345 0 90) (size 0.318 0.36) (layers "F.Paste") (roundrect_rratio 0.25))
  (pad "1" smd roundrect (at -0.32 0 90) (size 0.46 0.4) (layers "F.Cu" "F.Mask") (roundrect_rratio 0.25) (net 50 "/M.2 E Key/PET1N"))
  (pad "2" smd roundrect (at 0.32 0 90) (size 0.46 0.4) (layers "F.Cu" "F.Mask") (roundrect_rratio 0.25) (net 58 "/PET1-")))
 (gr_line (start 98.76 154.95) (end 94.76 154.95) (stroke (width 0.1) (type default)) (layer "Edge.Cuts"))
 (gr_line (start 124.76 128.95) (end 94.76 128.95) (stroke (width 0.1) (type default)) (layer "Edge.Cuts"))
 (gr_line (start 120.76 154.95) (end 124.76 154.95) (stroke (width 0.1) (type default)) (layer "Edge.Cuts"))
 (gr_line (start 94.76 128.95) (end 94.76 154.95) (stroke (width 0.1) (type default)) (layer "Edge.Cuts"))
 (gr_line (start 124.76 154.95) (end 124.76 128.95) (stroke (width 0.1) (type default)) (layer "Edge.Cuts"))
 (segment (start 102.985 156.499999) (end 102.985 154.970001) (width 0.2) (layer "F.Cu") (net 48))
 (segment (start 103.01 156.524999) (end 102.985 156.499999) (width 0.2) (layer "F.Cu") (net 48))
 (segment (start 102.985 154.970001) (end 103.11 154.845001) (width 0.2) (layer "F.Cu") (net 48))
 (segment (start 103.11 154.845001) (end 103.11 154.5) (width 0.2) (layer "F.Cu") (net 48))
 (segment (start 103.01 157.8) (end 103.01 156.524999) (width 0.2) (layer "F.Cu") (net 48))
 (segment (start 102.41 154.845001) (end 102.41 154.5) (width 0.2) (layer "F.Cu") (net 50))
 (segment (start 102.51 156.524999) (end 102.535 156.499999) (width 0.2) (layer "F.Cu") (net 50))
 (segment (start 102.535 154.970001) (end 102.41 154.845001) (width 0.2) (layer "F.Cu") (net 50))
 (segment (start 102.51 157.8) (end 102.51 156.524999) (width 0.2) (layer "F.Cu") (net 50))
 (segment (start 102.535 156.499999) (end 102.535 154.970001) (width 0.2) (layer "F.Cu") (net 50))
 (segment (start 109.01 157.8) (end 109.01 156.524999) (width 0.2) (layer "F.Cu") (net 28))
 (segment (start 108.985 154.970001) (end 109.11 154.845001) (width 0.2) (layer "F.Cu") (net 28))
 (segment (start 109.01 156.524999) (end 108.985 156.499999) (width 0.2) (layer "F.Cu") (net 28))
 (segment (start 109.11 154.845001) (end 109.11 154.5) (width 0.2) (layer "F.Cu") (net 28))
 (segment (start 108.985 156.499999) (end 108.985 154.970001) (width 0.2) (layer "F.Cu") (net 28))
 (segment (start 108.535 156.499999) (end 108.535 154.970001) (width 0.2) (layer "F.Cu") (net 30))
 (segment (start 108.51 156.524999) (end 108.535 156.499999) (width 0.2) (layer "F.Cu") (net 30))
 (segment (start 108.535 154.970001) (end 108.41 154.845001) (width 0.2) (layer "F.Cu") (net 30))
 (segment (start 108.51 157.8) (end 108.51 156.524999) (width 0.2) (layer "F.Cu") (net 30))
 (segment (start 108.41 154.845001) (end 108.41 154.5) (width 0.2) (layer "F.Cu") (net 30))
 (via (at 114.76 155.46) (size 0.6) (drill 0.3) (layers "F.Cu" "B.Cu") (free yes) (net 1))
 (segment (start 114.76 155.46) (end 114.76 157.55) (width 0.2) (layer "B.Cu") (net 1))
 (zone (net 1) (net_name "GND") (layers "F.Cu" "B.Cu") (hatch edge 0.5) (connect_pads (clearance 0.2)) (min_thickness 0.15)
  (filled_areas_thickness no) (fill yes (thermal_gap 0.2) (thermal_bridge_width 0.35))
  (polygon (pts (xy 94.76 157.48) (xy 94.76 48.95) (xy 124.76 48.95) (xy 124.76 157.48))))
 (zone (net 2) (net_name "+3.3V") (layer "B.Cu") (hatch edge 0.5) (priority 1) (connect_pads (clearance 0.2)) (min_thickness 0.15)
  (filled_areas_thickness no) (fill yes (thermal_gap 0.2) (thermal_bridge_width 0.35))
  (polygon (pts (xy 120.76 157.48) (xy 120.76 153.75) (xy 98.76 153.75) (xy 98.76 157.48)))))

